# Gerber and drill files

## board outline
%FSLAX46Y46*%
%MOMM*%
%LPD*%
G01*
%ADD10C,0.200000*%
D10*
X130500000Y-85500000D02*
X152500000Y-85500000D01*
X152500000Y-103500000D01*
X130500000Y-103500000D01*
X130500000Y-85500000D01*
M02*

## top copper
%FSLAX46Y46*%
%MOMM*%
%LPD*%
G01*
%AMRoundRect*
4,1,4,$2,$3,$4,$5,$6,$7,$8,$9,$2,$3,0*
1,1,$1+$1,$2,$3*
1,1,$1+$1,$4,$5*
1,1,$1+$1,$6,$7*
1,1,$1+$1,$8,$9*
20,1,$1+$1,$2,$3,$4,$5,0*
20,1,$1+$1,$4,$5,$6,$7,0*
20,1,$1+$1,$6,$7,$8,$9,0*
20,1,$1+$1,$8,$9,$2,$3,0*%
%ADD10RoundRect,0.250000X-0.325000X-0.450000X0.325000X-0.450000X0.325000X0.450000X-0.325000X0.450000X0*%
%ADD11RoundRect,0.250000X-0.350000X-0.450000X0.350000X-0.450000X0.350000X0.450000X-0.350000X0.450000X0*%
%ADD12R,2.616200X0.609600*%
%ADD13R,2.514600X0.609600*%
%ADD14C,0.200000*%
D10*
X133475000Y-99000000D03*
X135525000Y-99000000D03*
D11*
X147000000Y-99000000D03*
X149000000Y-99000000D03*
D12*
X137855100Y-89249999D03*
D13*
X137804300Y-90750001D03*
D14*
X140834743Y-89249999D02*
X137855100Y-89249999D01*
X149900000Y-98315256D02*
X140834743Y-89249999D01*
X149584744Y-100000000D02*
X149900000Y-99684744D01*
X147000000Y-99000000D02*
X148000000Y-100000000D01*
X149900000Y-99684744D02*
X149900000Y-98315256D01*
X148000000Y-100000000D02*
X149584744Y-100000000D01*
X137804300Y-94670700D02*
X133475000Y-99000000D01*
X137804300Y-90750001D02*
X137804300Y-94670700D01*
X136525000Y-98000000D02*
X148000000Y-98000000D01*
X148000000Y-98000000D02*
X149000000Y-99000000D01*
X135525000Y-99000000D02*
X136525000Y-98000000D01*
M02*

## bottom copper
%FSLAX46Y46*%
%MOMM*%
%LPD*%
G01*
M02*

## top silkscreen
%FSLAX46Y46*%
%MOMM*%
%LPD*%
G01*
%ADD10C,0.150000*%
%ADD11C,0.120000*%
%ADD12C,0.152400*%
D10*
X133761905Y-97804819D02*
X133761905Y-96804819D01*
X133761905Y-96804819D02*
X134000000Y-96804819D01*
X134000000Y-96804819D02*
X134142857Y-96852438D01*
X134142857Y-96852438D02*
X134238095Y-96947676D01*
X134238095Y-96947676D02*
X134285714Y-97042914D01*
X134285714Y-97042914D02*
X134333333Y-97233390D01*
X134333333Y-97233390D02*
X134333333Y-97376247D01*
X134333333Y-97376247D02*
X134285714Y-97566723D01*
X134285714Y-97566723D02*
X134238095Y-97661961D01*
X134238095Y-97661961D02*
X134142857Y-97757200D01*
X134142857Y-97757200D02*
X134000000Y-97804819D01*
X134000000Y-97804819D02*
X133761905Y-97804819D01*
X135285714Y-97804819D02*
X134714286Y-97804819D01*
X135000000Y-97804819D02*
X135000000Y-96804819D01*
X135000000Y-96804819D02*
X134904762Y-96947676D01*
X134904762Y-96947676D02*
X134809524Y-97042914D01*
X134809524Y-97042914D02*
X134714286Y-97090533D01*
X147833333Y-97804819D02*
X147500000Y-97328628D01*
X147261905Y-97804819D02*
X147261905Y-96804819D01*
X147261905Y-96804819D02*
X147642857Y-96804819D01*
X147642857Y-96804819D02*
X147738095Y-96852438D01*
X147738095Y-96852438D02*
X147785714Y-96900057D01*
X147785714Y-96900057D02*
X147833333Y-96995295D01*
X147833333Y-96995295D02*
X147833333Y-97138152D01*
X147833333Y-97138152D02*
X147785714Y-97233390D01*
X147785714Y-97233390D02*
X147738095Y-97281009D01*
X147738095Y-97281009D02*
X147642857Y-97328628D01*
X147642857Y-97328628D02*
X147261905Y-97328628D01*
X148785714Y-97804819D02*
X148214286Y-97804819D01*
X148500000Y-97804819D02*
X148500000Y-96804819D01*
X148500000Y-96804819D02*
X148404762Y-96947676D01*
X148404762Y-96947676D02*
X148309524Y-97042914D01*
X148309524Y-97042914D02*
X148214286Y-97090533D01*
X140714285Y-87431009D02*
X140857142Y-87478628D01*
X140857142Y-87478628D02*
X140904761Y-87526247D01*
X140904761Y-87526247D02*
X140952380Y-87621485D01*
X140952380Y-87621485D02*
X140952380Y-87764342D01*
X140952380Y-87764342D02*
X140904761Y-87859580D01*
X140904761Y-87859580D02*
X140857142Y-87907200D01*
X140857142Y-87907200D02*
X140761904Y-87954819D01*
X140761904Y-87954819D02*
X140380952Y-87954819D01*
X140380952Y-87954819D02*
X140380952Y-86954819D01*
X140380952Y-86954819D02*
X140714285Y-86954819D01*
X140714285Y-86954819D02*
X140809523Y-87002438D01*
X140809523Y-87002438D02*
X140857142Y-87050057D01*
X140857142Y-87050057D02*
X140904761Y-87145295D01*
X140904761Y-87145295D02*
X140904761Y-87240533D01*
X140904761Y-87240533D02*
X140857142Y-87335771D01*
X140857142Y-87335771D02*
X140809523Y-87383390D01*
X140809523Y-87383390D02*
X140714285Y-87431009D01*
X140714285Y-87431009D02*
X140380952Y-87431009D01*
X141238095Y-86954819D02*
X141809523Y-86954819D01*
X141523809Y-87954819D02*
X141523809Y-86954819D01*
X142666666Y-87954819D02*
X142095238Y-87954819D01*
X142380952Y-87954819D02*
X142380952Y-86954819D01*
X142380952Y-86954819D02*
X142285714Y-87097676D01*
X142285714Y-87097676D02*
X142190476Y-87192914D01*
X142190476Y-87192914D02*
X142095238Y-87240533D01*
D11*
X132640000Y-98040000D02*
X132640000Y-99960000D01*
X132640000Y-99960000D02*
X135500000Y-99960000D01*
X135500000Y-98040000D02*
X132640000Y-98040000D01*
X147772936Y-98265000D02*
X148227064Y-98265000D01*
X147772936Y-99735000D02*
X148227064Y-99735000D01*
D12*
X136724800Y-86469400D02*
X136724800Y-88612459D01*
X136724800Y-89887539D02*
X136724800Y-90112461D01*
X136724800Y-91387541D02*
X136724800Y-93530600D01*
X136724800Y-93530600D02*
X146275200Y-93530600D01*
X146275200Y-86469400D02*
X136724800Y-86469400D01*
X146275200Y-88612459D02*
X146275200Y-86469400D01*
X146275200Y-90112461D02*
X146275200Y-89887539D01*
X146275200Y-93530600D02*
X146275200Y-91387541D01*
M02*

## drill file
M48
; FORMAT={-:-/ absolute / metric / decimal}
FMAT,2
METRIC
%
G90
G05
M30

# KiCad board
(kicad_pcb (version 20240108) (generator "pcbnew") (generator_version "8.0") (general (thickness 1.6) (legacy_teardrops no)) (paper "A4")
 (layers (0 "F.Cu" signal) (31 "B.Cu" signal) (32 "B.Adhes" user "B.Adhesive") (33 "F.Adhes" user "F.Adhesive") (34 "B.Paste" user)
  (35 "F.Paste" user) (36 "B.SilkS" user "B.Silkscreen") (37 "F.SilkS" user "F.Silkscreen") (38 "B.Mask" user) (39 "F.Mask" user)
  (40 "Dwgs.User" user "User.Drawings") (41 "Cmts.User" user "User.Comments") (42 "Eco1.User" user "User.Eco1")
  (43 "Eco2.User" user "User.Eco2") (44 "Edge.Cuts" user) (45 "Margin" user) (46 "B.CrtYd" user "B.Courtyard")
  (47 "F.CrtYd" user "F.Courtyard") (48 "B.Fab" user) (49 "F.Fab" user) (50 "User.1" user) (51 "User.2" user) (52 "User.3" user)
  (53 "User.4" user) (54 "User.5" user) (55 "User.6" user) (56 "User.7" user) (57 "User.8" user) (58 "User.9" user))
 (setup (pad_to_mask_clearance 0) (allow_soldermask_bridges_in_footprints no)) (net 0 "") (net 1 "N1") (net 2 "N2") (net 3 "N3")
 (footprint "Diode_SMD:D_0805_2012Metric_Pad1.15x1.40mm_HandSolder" (layer "F.Cu") (at 134.5 99)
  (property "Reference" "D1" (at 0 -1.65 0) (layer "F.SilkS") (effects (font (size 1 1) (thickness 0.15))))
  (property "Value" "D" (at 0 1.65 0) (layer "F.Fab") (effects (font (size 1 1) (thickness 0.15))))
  (fp_line (start -1.86 -0.96) (end -1.86 0.96) (stroke (width 0.12) (type solid)) (layer "F.SilkS"))
  (fp_line (start -1.86 0.96) (end 1 0.96) (stroke (width 0.12) (type solid)) (layer "F.SilkS"))
  (fp_line (start 1 -0.96) (end -1.86 -0.96) (stroke (width 0.12) (type solid)) (layer "F.SilkS"))
  (pad "1" smd roundrect (at -1.025 0) (size 1.15 1.4) (layers "F.Cu" "F.Paste" "F.Mask") (roundrect_rratio 0.217391) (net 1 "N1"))
  (pad "2" smd roundrect (at 1.025 0) (size 1.15 1.4) (layers "F.Cu" "F.Paste" "F.Mask") (roundrect_rratio 0.217391) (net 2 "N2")))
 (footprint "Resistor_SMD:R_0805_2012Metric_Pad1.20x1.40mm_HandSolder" (layer "F.Cu") (at 148 99)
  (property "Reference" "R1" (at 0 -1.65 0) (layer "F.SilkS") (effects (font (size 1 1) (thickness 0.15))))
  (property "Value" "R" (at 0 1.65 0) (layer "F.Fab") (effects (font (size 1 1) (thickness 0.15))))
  (fp_line (start -0.227064 -0.735) (end 0.227064 -0.735) (stroke (width 0.12) (type solid)) (layer "F.SilkS"))
  (fp_line (start -0.227064 0.735) (end 0.227064 0.735) (stroke (width 0.12) (type solid)) (layer "F.SilkS"))
  (pad "1" smd roundrect (at -1 0) (size 1.2 1.4) (layers "F.Cu" "F.Paste" "F.Mask") (roundrect_rratio 0.208333) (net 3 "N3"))
  (pad "2" smd roundrect (at 1 0) (size 1.2 1.4) (layers "F.Cu" "F.Paste" "F.Mask") (roundrect_rratio 0.208333) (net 2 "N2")))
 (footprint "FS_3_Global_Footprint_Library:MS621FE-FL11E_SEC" (layer "F.Cu") (at 141.5 90)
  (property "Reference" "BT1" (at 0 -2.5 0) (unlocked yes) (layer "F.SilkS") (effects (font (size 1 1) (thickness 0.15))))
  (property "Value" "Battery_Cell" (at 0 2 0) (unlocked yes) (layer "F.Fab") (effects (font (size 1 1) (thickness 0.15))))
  (fp_line (start -4.7752 -3.5306) (end -4.7752 -1.387541) (stroke (width 0.1524) (type solid)) (layer "F.SilkS"))
  (fp_line (start -4.7752 -0.112461) (end -4.7752 0.112461) (stroke (width 0.1524) (type solid)) (layer "F.SilkS"))
  (fp_line (start -4.7752 1.387541) (end -4.7752 3.5306) (stroke (width 0.1524) (type solid)) (layer "F.SilkS"))
  (fp_line (start -4.7752 3.5306) (end 4.7752 3.5306) (stroke (width 0.1524) (type solid)) (layer "F.SilkS"))
  (fp_line (start 4.7752 -3.5306) (end -4.7752 -3.5306) (stroke (width 0.1524) (type solid)) (layer "F.SilkS"))
  (fp_line (start 4.7752 -1.387541) (end 4.7752 -3.5306) (stroke (width 0.1524) (type solid)) (layer "F.SilkS"))
  (fp_line (start 4.7752 0.112461) (end 4.7752 -0.112461) (stroke (width 0.1524) (type solid)) (layer "F.SilkS"))
  (fp_line (start 4.7752 3.5306) (end 4.7752 1.387541) (stroke (width 0.1524) (type solid)) (layer "F.SilkS"))
  (pad "1" smd rect (at -3.6449 -0.750001) (size 2.6162 0.6096) (layers "F.Cu" "F.Paste" "F.Mask") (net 3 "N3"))
  (pad "2" smd rect (at -3.6957 0.750001) (size 2.5146 0.6096) (layers "F.Cu" "F.Paste" "F.Mask") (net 1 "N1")))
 (gr_rect (start 130.5 85.5) (end 152.5 103.5) (stroke (width 0.2) (type default)) (fill none) (layer "Edge.Cuts"))
 (segment (start 140.834743 89.249999) (end 137.8551 89.249999) (width 0.2) (layer "F.Cu") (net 3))
 (segment (start 149.9 98.315256) (end 140.834743 89.249999) (width 0.2) (layer "F.Cu") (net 3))
 (segment (start 149.584744 100) (end 149.9 99.684744) (width 0.2) (layer "F.Cu") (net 3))
 (segment (start 147 99) (end 148 100) (width 0.2) (layer "F.Cu") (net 3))
 (segment (start 149.9 99.684744) (end 149.9 98.315256) (width 0.2) (layer "F.Cu") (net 3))
 (segment (start 148 100) (end 149.584744 100) (width 0.2) (layer "F.Cu") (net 3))
 (segment (start 137.8043 94.6707) (end 133.475 99) (width 0.2) (layer "F.Cu") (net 1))
 (segment (start 137.8043 90.750001) (end 137.8043 94.6707) (width 0.2) (layer "F.Cu") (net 1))
 (segment (start 136.525 98) (end 148 98) (width 0.2) (layer "F.Cu") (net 2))
 (segment (start 148 98) (end 149 99) (width 0.2) (layer "F.Cu") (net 2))
 (segment (start 135.525 99) (end 136.525 98) (width 0.2) (layer "F.Cu") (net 2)))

